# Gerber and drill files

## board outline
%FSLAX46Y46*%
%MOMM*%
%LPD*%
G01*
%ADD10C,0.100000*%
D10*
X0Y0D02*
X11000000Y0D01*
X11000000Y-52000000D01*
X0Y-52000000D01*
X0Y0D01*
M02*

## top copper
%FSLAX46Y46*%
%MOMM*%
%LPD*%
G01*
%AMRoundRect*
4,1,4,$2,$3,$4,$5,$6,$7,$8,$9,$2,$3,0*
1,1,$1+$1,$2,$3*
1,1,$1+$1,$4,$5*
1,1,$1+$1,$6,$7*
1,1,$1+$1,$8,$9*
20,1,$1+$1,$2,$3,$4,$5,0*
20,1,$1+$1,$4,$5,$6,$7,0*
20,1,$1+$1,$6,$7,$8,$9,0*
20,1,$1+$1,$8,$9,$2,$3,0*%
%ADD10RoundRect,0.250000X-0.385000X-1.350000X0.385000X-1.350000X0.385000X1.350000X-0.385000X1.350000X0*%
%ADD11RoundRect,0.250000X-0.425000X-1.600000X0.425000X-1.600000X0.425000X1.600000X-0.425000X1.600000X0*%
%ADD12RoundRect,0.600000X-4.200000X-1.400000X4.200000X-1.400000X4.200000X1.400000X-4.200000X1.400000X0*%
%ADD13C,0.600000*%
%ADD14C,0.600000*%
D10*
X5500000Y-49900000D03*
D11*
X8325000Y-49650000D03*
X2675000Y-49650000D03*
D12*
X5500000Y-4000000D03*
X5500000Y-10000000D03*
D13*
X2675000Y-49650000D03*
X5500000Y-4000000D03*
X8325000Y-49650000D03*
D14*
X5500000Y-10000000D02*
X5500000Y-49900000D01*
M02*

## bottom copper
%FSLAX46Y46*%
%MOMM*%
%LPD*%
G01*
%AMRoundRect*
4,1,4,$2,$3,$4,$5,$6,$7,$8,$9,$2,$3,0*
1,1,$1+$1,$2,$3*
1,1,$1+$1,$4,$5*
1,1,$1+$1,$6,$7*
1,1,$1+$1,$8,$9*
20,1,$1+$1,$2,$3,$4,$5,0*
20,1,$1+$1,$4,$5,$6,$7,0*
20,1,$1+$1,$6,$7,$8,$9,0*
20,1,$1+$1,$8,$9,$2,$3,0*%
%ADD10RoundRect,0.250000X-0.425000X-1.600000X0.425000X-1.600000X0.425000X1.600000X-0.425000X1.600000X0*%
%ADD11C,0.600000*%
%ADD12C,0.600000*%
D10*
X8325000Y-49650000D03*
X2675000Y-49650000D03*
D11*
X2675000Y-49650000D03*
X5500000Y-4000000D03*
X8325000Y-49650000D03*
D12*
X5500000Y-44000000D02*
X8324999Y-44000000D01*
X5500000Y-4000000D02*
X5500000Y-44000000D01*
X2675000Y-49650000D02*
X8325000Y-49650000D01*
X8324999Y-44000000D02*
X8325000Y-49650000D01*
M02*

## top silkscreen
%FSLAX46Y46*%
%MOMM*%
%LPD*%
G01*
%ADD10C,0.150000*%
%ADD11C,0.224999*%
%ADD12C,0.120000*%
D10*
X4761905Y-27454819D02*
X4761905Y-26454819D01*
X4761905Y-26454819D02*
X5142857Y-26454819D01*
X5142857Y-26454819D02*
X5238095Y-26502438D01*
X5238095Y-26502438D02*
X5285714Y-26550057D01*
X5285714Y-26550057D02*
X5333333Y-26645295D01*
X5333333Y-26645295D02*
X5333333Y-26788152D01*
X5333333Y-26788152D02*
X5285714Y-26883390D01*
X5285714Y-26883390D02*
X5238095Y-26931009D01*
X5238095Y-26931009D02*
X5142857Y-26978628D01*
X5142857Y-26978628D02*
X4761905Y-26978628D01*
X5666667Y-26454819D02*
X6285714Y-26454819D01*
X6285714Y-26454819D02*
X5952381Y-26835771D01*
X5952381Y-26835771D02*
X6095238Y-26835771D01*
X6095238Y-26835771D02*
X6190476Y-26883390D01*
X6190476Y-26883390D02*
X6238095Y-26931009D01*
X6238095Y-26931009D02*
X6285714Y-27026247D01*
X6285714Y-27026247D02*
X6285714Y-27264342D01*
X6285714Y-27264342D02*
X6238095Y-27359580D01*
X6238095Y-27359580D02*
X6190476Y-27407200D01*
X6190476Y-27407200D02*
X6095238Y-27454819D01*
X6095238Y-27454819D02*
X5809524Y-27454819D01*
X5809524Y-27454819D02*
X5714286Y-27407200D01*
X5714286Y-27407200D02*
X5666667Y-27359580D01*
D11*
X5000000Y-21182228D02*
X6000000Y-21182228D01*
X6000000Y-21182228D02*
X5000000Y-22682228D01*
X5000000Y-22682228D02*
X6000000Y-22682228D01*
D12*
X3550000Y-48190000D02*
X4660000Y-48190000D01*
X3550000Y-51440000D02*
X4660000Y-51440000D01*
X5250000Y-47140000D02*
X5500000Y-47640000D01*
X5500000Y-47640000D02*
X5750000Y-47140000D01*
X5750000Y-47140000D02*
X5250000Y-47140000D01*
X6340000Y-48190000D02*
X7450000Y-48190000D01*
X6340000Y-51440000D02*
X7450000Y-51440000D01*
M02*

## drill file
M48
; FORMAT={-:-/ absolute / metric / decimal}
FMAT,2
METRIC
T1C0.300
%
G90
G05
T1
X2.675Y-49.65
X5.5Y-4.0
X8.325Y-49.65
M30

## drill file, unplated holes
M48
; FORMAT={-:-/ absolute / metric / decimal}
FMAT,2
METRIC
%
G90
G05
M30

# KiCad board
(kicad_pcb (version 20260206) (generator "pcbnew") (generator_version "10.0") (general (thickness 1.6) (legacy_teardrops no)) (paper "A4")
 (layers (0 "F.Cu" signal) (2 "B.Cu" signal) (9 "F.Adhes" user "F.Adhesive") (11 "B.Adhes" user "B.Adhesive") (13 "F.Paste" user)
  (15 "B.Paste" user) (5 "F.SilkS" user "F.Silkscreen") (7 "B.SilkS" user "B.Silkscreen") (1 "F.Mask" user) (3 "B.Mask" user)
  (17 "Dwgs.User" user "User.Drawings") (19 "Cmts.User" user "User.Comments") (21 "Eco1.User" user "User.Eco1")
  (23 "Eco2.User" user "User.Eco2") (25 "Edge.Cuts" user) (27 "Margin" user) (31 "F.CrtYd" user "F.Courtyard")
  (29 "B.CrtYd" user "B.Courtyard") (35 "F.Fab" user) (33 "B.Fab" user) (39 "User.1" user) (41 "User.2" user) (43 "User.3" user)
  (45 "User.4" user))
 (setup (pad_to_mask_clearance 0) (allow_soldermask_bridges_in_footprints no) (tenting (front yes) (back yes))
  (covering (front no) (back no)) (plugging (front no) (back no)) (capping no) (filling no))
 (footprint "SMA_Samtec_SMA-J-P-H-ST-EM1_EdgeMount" (layer "F.Cu") (at 5.5 49.9 -90)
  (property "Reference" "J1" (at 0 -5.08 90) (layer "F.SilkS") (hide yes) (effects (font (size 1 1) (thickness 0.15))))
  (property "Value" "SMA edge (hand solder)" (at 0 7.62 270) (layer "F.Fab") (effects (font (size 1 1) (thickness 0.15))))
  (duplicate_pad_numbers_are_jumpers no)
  (fp_line (start -1.71 1.95) (end -1.71 0.84) (stroke (width 0.12) (type solid)) (layer "F.SilkS"))
  (fp_line (start 1.54 1.95) (end 1.54 0.84) (stroke (width 0.12) (type solid)) (layer "F.SilkS"))
  (fp_line (start -2.76 0.25) (end -2.26 0) (stroke (width 0.12) (type solid)) (layer "F.SilkS"))
  (fp_line (start -2.26 0) (end -2.76 -0.25) (stroke (width 0.12) (type solid)) (layer "F.SilkS"))
  (fp_line (start -2.76 -0.25) (end -2.76 0.25) (stroke (width 0.12) (type solid)) (layer "F.SilkS"))
  (fp_line (start -1.71 -0.84) (end -1.71 -1.95) (stroke (width 0.12) (type solid)) (layer "F.SilkS"))
  (fp_line (start 1.54 -0.84) (end 1.54 -1.95) (stroke (width 0.12) (type solid)) (layer "F.SilkS"))
  (pad "1" smd roundrect (at 0 0) (size 1.27 3.2) (layers "F.Cu" "F.Mask") (roundrect_rratio 0.1968503937) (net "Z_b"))
  (pad "2" smd roundrect (at -0.25 -2.825) (size 1.35 3.7) (layers "F.Cu" "F.Mask") (roundrect_rratio 0.1851851852) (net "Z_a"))
  (pad "2" smd roundrect (at -0.25 -2.825) (size 1.35 3.7) (layers "B.Cu" "B.Mask") (roundrect_rratio 0.1851851852) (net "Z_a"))
  (pad "2" smd roundrect (at -0.25 2.825) (size 1.35 3.7) (layers "F.Cu" "F.Mask") (roundrect_rratio 0.1851851852) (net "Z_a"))
  (pad "2" smd roundrect (at -0.25 2.825) (size 1.35 3.7) (layers "B.Cu" "B.Mask") (roundrect_rratio 0.1851851852) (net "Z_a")))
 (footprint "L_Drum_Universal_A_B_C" (layer "F.Cu") (at 5.5 7)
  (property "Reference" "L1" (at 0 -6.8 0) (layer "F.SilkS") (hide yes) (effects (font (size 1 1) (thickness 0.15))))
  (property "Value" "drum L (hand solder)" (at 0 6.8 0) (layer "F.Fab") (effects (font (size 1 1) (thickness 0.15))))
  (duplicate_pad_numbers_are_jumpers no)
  (pad "1" smd roundrect (at 0 -3) (size 9.6 4) (layers "F.Cu" "F.Mask" "F.Paste") (roundrect_rratio 0.15) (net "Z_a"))
  (pad "2" smd roundrect (at 0 3) (size 9.6 4) (layers "F.Cu" "F.Mask" "F.Paste") (roundrect_rratio 0.15) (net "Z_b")))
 (gr_rect (start 0 0) (end 11 52) (stroke (width 0.1) (type default)) (fill no) (layer "Edge.Cuts"))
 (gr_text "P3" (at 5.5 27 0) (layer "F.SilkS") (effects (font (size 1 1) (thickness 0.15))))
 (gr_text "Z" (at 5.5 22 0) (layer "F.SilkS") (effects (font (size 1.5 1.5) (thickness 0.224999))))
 (via (at 2.675 49.65) (size 0.6) (drill 0.3) (layers "F.Cu" "B.Cu") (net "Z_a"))
 (via (at 5.5 4) (size 0.6) (drill 0.3) (layers "F.Cu" "B.Cu") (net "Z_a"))
 (via (at 8.325 49.65) (size 0.6) (drill 0.3) (layers "F.Cu" "B.Cu") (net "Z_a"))
 (segment (start 5.5 44) (end 8.324999 44) (width 0.6) (layer "B.Cu") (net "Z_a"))
 (segment (start 5.5 4) (end 5.5 44) (width 0.6) (layer "B.Cu") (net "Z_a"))
 (segment (start 2.675 49.65) (end 8.325 49.65) (width 0.6) (layer "B.Cu") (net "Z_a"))
 (segment (start 8.324999 44) (end 8.325 49.65) (width 0.6) (layer "B.Cu") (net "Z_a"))
 (segment (start 5.5 10) (end 5.5 49.9) (width 0.6) (layer "F.Cu") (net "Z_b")))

